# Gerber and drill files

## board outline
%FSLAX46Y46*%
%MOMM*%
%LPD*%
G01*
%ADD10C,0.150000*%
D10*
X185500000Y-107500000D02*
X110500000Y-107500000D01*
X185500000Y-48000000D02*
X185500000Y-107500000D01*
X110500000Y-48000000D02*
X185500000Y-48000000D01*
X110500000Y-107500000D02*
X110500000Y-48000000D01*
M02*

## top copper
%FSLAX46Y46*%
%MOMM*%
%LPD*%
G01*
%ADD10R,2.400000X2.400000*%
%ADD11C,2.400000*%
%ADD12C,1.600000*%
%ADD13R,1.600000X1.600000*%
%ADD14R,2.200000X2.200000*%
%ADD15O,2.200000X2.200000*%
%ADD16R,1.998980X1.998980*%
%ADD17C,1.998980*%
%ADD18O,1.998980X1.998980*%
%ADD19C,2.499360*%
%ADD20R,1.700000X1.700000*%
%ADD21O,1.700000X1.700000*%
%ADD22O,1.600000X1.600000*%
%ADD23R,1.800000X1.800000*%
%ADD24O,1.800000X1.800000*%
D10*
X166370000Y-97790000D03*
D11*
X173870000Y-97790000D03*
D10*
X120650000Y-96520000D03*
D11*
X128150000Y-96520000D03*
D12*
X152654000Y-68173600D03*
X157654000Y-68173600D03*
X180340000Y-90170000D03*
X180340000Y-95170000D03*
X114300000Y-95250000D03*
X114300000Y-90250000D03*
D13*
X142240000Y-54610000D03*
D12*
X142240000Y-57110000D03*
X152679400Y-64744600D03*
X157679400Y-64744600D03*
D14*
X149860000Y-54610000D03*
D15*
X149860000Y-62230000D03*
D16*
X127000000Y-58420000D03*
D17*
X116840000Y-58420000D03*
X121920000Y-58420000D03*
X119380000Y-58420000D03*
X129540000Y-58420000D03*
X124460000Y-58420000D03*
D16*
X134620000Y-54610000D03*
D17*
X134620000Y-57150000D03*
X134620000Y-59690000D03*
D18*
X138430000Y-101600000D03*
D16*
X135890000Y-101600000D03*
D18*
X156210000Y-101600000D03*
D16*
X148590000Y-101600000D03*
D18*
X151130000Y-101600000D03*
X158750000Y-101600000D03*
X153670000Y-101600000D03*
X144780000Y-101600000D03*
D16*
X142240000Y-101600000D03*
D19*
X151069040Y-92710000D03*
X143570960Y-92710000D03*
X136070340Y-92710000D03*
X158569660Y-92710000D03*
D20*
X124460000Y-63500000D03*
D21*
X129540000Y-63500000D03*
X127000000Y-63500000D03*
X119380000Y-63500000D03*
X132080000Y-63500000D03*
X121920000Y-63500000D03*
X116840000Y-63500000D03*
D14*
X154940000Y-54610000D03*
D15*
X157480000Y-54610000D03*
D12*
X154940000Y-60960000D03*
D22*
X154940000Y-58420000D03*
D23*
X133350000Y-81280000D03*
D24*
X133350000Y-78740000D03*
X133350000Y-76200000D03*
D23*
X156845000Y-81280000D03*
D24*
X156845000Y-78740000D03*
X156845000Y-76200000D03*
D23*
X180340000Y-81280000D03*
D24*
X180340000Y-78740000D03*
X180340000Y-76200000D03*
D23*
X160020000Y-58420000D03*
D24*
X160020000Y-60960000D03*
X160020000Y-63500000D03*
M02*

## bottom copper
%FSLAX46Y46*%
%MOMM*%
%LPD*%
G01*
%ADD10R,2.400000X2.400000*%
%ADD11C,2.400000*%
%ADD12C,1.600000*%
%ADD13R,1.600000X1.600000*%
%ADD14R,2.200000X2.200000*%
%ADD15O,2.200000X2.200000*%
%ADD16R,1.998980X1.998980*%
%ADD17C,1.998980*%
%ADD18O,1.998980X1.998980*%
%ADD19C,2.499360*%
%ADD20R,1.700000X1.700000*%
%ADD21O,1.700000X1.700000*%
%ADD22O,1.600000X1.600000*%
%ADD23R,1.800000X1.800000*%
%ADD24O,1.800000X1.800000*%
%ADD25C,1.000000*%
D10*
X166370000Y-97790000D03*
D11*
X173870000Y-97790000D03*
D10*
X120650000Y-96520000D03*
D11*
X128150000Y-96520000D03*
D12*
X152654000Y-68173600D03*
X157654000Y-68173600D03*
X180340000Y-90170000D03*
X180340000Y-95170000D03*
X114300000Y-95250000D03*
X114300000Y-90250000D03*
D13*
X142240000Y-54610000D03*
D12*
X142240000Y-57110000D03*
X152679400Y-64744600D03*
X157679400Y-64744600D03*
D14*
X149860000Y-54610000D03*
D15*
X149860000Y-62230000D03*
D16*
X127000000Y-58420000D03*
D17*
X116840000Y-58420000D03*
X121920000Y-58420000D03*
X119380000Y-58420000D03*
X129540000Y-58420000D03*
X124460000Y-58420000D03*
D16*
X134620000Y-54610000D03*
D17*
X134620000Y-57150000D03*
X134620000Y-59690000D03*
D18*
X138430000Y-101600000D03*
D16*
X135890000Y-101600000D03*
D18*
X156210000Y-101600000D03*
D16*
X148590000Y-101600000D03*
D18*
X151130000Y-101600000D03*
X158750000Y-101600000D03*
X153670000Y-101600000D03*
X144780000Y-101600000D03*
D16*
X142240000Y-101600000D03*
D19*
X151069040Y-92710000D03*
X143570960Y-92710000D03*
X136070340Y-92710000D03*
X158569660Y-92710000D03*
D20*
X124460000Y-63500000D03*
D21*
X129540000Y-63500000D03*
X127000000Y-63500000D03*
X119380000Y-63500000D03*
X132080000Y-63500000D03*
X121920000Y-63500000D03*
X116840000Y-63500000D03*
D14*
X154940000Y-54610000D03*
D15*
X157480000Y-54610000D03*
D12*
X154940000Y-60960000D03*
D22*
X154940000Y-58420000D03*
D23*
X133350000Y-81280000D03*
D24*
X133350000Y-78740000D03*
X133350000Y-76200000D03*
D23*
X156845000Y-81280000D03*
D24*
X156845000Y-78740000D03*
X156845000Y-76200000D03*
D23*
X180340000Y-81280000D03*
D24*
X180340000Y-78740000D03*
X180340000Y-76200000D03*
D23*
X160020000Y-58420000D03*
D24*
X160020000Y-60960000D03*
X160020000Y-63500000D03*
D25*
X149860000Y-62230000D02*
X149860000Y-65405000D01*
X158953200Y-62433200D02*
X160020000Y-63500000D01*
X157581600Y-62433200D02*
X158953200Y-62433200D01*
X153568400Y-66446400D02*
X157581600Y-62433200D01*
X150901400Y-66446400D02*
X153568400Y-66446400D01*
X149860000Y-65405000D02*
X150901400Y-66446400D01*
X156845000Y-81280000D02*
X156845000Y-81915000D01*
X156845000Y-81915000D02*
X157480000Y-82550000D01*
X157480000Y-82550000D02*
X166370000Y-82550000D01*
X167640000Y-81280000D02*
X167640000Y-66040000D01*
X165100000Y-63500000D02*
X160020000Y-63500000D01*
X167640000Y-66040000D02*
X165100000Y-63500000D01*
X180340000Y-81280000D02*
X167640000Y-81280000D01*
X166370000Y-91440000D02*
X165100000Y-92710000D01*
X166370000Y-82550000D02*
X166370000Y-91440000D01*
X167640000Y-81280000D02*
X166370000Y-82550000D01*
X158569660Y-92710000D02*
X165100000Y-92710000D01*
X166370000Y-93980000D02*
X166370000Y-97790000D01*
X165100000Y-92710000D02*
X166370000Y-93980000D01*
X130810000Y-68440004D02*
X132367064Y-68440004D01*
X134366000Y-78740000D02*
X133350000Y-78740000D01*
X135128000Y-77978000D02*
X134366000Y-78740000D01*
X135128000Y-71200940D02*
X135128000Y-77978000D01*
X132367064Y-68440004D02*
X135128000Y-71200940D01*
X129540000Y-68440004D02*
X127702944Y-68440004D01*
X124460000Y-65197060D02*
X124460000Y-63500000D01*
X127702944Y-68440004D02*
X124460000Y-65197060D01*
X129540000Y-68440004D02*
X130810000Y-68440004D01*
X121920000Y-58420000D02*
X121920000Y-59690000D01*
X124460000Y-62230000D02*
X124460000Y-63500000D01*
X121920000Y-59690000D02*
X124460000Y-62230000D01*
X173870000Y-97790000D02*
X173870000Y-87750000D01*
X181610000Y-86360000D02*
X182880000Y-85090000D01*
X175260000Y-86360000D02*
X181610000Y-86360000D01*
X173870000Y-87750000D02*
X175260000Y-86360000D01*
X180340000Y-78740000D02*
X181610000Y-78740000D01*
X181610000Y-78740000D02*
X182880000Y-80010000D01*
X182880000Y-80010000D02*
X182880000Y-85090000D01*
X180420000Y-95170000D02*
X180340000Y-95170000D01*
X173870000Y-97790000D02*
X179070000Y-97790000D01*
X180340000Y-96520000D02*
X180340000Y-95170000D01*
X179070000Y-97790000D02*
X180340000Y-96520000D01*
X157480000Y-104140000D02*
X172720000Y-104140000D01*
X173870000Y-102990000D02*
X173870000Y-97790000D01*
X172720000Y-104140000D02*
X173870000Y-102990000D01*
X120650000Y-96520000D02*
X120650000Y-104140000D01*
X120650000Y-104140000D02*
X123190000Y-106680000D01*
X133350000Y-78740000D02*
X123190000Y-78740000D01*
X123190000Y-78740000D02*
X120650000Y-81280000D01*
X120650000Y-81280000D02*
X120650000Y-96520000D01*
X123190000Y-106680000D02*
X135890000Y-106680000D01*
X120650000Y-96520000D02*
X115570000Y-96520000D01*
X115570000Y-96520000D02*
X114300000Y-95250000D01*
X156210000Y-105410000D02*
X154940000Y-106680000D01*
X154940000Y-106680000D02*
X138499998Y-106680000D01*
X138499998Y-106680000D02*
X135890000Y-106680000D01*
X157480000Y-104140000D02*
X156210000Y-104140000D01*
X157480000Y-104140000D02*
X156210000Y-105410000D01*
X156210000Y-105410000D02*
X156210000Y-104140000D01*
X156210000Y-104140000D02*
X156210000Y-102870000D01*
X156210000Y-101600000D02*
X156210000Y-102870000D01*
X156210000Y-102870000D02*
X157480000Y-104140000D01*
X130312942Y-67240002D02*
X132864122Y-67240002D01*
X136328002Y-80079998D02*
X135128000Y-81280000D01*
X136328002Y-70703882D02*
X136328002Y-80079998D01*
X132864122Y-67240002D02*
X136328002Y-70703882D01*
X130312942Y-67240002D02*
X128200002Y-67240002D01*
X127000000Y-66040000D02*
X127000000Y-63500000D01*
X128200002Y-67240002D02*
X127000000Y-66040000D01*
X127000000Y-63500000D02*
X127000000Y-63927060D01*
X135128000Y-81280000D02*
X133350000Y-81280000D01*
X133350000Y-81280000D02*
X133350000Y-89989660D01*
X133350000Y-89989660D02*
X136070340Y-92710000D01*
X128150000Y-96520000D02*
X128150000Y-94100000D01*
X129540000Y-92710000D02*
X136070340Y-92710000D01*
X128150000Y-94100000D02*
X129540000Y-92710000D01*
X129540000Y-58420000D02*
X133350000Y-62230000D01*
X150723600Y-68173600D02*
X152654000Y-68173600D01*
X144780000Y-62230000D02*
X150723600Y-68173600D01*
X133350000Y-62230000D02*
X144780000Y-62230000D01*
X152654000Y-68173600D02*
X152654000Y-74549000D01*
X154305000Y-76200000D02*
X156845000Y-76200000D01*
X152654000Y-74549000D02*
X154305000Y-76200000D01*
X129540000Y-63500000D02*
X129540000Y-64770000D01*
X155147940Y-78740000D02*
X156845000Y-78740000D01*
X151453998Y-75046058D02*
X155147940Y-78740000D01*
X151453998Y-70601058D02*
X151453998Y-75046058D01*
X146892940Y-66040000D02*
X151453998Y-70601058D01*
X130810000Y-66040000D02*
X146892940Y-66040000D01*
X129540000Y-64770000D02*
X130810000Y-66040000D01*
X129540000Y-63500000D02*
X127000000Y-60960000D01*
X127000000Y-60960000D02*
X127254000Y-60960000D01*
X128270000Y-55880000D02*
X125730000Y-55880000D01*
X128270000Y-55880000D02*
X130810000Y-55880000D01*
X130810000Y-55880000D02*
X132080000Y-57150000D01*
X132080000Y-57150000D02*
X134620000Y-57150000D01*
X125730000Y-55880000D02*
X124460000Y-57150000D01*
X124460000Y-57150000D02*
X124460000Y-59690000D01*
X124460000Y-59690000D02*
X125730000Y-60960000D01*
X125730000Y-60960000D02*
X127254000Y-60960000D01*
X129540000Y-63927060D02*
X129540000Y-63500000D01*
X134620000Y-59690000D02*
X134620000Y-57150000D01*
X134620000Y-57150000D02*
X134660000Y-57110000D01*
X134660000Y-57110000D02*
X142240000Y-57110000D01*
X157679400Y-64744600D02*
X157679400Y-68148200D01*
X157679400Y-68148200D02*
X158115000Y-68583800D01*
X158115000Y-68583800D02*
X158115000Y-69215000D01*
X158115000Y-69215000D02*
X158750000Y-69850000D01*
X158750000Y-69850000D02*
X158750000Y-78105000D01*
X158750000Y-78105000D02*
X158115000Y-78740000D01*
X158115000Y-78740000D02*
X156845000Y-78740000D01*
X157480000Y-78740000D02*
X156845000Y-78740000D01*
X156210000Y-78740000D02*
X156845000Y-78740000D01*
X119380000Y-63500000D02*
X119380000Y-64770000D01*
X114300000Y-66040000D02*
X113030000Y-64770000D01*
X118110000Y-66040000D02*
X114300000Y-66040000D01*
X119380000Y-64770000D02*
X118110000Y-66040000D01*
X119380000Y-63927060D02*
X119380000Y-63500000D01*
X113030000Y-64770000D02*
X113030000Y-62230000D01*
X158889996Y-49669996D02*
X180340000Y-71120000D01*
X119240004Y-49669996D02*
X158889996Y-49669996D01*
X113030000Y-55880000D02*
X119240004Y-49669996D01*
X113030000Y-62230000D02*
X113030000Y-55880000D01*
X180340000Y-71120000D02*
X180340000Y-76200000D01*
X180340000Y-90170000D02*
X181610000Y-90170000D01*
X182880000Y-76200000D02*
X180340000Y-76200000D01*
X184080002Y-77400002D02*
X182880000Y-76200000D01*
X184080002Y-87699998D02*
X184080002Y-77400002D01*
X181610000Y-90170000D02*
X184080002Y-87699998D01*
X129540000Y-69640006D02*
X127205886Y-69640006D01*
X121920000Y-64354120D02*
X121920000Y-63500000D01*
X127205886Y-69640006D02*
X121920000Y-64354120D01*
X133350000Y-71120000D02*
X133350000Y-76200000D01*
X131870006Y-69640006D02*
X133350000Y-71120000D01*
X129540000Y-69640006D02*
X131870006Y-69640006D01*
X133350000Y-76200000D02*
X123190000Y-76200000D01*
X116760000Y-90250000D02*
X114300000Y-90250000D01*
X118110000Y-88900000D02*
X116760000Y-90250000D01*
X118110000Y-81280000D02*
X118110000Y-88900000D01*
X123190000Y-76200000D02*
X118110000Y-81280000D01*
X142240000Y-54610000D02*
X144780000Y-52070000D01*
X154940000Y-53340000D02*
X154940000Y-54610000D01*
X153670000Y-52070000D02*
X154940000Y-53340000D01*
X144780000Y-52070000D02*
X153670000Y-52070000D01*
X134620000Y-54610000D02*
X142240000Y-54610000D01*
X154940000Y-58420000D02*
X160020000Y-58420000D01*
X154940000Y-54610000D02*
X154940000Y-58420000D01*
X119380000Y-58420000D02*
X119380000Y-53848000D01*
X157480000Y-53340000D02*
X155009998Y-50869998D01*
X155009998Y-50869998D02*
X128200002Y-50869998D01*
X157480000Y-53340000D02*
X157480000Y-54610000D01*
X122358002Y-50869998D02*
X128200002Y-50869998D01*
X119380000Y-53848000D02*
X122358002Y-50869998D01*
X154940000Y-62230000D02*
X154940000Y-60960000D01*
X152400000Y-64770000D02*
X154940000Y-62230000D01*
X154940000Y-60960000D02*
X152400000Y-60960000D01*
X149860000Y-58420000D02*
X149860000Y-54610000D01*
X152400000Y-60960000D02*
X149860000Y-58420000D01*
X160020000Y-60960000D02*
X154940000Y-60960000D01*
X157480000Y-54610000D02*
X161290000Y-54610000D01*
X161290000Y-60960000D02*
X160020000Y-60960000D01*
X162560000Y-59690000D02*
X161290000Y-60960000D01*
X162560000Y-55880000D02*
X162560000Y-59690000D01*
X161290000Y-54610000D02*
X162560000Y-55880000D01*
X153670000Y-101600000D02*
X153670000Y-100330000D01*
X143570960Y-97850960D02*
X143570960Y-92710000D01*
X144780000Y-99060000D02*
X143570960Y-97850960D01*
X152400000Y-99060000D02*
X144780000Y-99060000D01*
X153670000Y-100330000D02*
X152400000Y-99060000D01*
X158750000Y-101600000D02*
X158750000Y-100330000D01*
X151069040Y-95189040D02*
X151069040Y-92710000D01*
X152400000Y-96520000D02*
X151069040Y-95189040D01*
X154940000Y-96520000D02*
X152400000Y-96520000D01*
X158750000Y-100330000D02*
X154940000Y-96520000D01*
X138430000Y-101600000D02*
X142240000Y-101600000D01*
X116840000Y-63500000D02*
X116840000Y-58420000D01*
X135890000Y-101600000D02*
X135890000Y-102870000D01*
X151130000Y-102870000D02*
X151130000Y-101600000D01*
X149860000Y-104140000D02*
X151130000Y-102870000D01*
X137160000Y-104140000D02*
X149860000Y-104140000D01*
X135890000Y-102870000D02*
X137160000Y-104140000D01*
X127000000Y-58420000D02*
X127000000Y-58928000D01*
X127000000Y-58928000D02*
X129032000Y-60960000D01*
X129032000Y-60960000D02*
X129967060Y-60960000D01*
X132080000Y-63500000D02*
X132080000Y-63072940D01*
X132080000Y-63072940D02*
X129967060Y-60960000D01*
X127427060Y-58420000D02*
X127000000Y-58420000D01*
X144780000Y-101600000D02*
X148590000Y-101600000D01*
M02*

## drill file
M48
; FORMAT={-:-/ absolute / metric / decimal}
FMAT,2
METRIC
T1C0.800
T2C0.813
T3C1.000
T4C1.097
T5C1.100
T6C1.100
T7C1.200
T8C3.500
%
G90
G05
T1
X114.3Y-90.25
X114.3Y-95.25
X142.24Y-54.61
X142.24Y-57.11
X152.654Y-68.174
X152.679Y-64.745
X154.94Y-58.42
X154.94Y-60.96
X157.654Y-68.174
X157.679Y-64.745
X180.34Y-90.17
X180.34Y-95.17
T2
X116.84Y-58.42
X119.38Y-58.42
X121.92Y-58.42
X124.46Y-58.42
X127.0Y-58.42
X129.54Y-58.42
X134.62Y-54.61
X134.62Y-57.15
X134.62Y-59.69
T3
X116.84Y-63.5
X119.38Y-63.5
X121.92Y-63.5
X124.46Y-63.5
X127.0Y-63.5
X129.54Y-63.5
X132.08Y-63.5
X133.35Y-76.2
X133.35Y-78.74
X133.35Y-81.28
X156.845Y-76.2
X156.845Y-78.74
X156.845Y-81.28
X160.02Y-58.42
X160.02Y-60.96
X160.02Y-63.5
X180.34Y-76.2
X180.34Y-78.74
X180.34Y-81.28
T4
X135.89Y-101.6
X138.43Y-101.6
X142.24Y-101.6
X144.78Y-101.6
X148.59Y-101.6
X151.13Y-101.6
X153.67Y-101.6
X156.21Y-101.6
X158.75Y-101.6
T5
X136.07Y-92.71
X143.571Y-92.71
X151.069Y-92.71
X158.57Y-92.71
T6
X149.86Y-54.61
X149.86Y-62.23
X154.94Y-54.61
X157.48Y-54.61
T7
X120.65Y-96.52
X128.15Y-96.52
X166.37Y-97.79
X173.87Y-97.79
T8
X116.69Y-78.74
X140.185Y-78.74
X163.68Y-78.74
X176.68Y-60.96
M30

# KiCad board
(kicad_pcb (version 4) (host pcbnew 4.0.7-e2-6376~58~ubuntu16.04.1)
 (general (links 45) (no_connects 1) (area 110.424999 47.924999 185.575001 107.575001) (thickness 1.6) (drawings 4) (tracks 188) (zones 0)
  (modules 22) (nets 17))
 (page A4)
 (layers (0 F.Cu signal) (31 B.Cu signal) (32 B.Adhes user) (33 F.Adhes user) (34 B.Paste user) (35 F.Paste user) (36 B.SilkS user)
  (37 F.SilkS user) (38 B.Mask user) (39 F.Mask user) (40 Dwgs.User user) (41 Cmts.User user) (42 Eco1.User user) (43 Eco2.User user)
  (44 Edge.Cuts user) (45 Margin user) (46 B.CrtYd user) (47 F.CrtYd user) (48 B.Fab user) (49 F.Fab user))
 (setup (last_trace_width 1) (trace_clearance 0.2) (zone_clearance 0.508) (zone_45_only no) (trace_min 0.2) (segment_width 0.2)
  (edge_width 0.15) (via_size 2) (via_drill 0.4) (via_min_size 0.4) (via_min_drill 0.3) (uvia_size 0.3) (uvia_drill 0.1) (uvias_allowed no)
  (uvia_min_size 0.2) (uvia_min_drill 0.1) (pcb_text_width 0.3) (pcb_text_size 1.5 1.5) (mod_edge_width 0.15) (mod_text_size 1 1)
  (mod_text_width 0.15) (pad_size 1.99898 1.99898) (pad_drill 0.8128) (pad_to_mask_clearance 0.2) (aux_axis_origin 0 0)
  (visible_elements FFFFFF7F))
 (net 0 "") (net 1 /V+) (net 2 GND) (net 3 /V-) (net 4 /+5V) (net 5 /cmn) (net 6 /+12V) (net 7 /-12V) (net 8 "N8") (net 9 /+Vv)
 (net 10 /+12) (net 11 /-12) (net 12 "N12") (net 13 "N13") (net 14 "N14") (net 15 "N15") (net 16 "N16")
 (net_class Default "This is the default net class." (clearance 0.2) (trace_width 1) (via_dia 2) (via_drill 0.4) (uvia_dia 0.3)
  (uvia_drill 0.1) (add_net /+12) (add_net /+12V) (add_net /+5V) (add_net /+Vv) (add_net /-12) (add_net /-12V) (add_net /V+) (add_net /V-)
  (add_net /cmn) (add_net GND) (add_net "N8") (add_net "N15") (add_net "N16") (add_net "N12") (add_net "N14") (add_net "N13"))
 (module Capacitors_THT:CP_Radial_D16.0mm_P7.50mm (layer F.Cu) (at 166.37 97.79)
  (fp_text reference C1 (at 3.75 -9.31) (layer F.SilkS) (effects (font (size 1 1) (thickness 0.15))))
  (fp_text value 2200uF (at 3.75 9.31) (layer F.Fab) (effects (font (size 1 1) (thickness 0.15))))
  (pad 1 thru_hole rect (at 0 0) (size 2.4 2.4) (drill 1.2) (layers *.Cu *.Mask) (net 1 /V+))
  (pad 2 thru_hole circle (at 7.5 0) (size 2.4 2.4) (drill 1.2) (layers *.Cu *.Mask) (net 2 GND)))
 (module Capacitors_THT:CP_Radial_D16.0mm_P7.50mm (layer F.Cu) (at 120.65 96.52)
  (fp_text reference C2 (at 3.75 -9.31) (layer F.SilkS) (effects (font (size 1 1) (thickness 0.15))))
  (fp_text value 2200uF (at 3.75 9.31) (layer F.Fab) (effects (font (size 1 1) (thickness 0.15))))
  (pad 1 thru_hole rect (at 0 0) (size 2.4 2.4) (drill 1.2) (layers *.Cu *.Mask) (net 2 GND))
  (pad 2 thru_hole circle (at 7.5 0) (size 2.4 2.4) (drill 1.2) (layers *.Cu *.Mask) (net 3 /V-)))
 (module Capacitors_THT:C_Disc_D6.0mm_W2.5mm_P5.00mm (layer F.Cu) (at 152.654 68.1736)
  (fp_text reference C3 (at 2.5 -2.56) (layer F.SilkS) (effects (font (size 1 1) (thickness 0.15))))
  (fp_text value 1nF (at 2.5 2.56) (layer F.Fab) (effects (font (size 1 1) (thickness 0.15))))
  (pad 1 thru_hole circle (at 0 0) (size 1.6 1.6) (drill 0.8) (layers *.Cu *.Mask) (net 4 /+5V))
  (pad 2 thru_hole circle (at 5 0) (size 1.6 1.6) (drill 0.8) (layers *.Cu *.Mask) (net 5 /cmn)))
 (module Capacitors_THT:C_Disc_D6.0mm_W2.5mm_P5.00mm (layer F.Cu) (at 180.34 90.17 270)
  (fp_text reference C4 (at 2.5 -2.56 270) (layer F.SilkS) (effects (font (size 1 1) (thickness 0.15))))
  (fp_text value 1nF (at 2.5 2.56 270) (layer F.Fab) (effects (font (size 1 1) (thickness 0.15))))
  (pad 1 thru_hole circle (at 0 0 270) (size 1.6 1.6) (drill 0.8) (layers *.Cu *.Mask) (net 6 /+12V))
  (pad 2 thru_hole circle (at 5 0 270) (size 1.6 1.6) (drill 0.8) (layers *.Cu *.Mask) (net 2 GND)))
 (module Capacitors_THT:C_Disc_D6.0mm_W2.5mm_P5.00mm (layer F.Cu) (at 114.3 95.25 90)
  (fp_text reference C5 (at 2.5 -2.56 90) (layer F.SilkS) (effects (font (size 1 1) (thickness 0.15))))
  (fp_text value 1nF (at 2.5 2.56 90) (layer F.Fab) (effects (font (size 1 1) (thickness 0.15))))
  (pad 1 thru_hole circle (at 0 0 90) (size 1.6 1.6) (drill 0.8) (layers *.Cu *.Mask) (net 2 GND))
  (pad 2 thru_hole circle (at 5 0 90) (size 1.6 1.6) (drill 0.8) (layers *.Cu *.Mask) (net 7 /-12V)))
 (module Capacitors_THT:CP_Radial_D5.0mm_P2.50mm (layer F.Cu) (at 142.24 54.61 270)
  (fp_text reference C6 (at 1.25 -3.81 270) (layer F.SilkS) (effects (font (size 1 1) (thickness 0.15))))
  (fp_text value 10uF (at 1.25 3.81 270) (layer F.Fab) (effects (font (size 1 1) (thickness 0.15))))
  (pad 1 thru_hole rect (at 0 0 270) (size 1.6 1.6) (drill 0.8) (layers *.Cu *.Mask) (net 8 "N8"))
  (pad 2 thru_hole circle (at 2.5 0 270) (size 1.6 1.6) (drill 0.8) (layers *.Cu *.Mask) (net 5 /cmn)))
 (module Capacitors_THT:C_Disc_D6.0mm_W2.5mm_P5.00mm (layer F.Cu) (at 152.6794 64.7446)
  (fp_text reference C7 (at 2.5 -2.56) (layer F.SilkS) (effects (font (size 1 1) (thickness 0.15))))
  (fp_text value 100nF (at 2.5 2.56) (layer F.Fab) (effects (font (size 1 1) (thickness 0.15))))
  (pad 1 thru_hole circle (at 0 0) (size 1.6 1.6) (drill 0.8) (layers *.Cu *.Mask) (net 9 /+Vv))
  (pad 2 thru_hole circle (at 5 0) (size 1.6 1.6) (drill 0.8) (layers *.Cu *.Mask) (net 5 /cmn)))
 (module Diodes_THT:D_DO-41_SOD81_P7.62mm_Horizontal (layer F.Cu) (at 149.86 54.61 270)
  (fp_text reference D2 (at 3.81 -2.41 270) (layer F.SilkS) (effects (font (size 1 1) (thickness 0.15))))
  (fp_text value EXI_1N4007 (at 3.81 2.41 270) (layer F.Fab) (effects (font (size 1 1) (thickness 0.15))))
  (pad 1 thru_hole rect (at 0 0 270) (size 2.2 2.2) (drill 1.1) (layers *.Cu *.Mask) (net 9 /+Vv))
  (pad 2 thru_hole oval (at 7.62 0 270) (size 2.2 2.2) (drill 1.1) (layers *.Cu *.Mask) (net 1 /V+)))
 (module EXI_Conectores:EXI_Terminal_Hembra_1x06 (layer F.Cu) (at 123.19 58.42 180)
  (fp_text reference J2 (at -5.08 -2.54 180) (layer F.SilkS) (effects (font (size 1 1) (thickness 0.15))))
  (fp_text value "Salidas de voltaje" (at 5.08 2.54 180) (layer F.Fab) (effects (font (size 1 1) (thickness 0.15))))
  (pad 1 thru_hole rect (at -3.81 0 180) (size 1.99898 1.99898) (drill 0.8128) (layers *.Cu *.Mask F.SilkS) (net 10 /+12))
  (pad 2 thru_hole circle (at 6.35 0 180) (size 1.99898 1.99898) (drill 0.8128) (layers *.Cu *.Mask F.SilkS) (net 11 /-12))
  (pad 3 thru_hole circle (at 1.27 0 180) (size 1.99898 1.99898) (drill 0.8128) (layers *.Cu *.Mask F.SilkS) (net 2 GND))
  (pad 4 thru_hole circle (at 3.81 0 180) (size 1.99898 1.99898) (drill 0.8128) (layers *.Cu *.Mask F.SilkS) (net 9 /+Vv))
  (pad 5 thru_hole circle (at -6.35 0 180) (size 1.99898 1.99898) (drill 0.8128) (layers *.Cu *.Mask F.SilkS) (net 4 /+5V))
  (pad 6 thru_hole circle (at -1.27 0 180) (size 1.99898 1.99898) (drill 0.8128) (layers *.Cu *.Mask F.SilkS) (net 5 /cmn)))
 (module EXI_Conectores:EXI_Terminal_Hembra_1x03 (layer F.Cu) (at 134.62 57.15 270)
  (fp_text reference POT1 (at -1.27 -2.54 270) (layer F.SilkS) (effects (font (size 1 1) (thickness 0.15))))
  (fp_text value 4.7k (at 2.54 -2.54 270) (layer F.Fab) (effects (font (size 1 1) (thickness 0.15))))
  (pad 1 thru_hole rect (at -2.54 0 270) (size 1.99898 1.99898) (drill 0.8128) (layers *.Cu *.Mask F.SilkS) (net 8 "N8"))
  (pad 2 thru_hole circle (at 0 0 270) (size 1.99898 1.99898) (drill 0.8128) (layers *.Cu *.Mask F.SilkS) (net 5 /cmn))
  (pad 3 thru_hole circle (at 2.54 0 270) (size 1.99898 1.99898) (drill 0.8128) (layers *.Cu *.Mask F.SilkS) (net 5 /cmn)))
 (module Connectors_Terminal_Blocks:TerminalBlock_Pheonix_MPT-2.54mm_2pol (layer F.Cu) (at 135.89 101.6)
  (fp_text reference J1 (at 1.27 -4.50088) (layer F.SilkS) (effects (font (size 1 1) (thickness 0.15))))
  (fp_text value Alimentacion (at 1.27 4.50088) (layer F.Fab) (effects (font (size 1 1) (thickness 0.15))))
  (pad 2 thru_hole oval (at 2.54 0) (size 1.99898 1.99898) (drill 1.09728) (layers *.Cu *.Mask) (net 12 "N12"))
  (pad 1 thru_hole rect (at 0 0) (size 1.99898 1.99898) (drill 1.09728) (layers *.Cu *.Mask) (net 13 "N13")))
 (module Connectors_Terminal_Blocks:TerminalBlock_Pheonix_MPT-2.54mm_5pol (layer F.Cu) (at 148.59 101.6)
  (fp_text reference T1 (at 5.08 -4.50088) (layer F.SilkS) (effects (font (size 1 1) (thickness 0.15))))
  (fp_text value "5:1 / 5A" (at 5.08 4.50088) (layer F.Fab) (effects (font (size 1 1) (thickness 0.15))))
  (pad 4 thru_hole oval (at 7.62 0 180) (size 1.99898 1.99898) (drill 1.09728) (layers *.Cu *.Mask) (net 2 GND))
  (pad 1 thru_hole rect (at 0 0 180) (size 1.99898 1.99898) (drill 1.09728) (layers *.Cu *.Mask) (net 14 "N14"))
  (pad 2 thru_hole oval (at 2.54 0 180) (size 1.99898 1.99898) (drill 1.09728) (layers *.Cu *.Mask) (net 13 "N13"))
  (pad 3 thru_hole oval (at 10.16 0 180) (size 1.99898 1.99898) (drill 1.09728) (layers *.Cu *.Mask) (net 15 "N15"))
  (pad 5 thru_hole oval (at 5.08 0 180) (size 1.99898 1.99898) (drill 1.09728) (layers *.Cu *.Mask) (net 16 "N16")))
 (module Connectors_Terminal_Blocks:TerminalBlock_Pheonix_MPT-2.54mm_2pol (layer F.Cu) (at 142.24 101.6)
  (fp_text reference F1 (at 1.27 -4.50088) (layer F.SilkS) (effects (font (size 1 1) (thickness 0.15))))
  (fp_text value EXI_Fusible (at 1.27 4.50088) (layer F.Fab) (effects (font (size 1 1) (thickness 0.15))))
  (pad 2 thru_hole oval (at 2.54 0) (size 1.99898 1.99898) (drill 1.09728) (layers *.Cu *.Mask) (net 14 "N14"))
  (pad 1 thru_hole rect (at 0 0) (size 1.99898 1.99898) (drill 1.09728) (layers *.Cu *.Mask) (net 12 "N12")))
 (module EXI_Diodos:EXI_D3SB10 (layer F.Cu) (at 147.32 92.71 180)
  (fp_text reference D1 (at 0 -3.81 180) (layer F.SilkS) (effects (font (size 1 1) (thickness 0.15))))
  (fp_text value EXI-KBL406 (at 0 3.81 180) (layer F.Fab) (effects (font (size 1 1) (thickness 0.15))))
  (pad 2 thru_hole circle (at -3.74904 0 180) (size 2.49936 2.49936) (drill 1.09982) (layers *.Cu *.Mask F.SilkS) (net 15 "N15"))
  (pad 3 thru_hole circle (at 3.74904 0 180) (size 2.49936 2.49936) (drill 1.09982) (layers *.Cu *.Mask F.SilkS) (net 16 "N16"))
  (pad 4 thru_hole circle (at 11.24966 0 180) (size 2.49936 2.49936) (drill 1.09982) (layers *.Cu *.Mask F.SilkS) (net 3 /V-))
  (pad 1 thru_hole circle (at -11.24966 0 180) (size 2.49936 2.49936) (drill 1.09982) (layers *.Cu *.Mask F.SilkS) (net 1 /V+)))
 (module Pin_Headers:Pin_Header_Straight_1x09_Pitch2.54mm (layer F.Cu) (at 137.16 63.5 270)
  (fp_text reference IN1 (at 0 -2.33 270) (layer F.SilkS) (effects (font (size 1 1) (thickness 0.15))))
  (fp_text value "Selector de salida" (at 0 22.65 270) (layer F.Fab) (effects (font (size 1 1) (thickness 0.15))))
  (pad 1 thru_hole rect (at 0 12.7 270) (size 1.7 1.7) (drill 1) (layers *.Cu *.Mask) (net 2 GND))
  (pad 2 thru_hole oval (at 0 7.62 270) (size 1.7 1.7) (drill 1) (layers *.Cu *.Mask) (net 5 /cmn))
  (pad 3 thru_hole oval (at 0 10.16 270) (size 1.7 1.7) (drill 1) (layers *.Cu *.Mask) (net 3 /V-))
  (pad 4 thru_hole oval (at 0 17.78 270) (size 1.7 1.7) (drill 1) (layers *.Cu *.Mask) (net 6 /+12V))
  (pad 5 thru_hole oval (at 0 5.08 270) (size 1.7 1.7) (drill 1) (layers *.Cu *.Mask) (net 10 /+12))
  (pad 7 thru_hole oval (at 0 15.24 270) (size 1.7 1.7) (drill 1) (layers *.Cu *.Mask) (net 7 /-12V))
  (pad 8 thru_hole oval (at 0 20.32 270) (size 1.7 1.7) (drill 1) (layers *.Cu *.Mask) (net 11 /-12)))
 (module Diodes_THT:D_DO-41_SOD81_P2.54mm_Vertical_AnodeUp (layer F.Cu) (at 154.94 54.61)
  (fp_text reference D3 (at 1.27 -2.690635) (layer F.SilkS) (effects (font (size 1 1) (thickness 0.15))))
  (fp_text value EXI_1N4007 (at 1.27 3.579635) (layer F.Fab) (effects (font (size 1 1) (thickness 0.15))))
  (pad 1 thru_hole rect (at 0 0) (size 2.2 2.2) (drill 1.1) (layers *.Cu *.Mask) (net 8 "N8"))
  (pad 2 thru_hole oval (at 2.54 0) (size 2.2 2.2) (drill 1.1) (layers *.Cu *.Mask) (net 9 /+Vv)))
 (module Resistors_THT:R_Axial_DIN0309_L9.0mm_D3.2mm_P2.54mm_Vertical (layer F.Cu) (at 154.94 60.96 90)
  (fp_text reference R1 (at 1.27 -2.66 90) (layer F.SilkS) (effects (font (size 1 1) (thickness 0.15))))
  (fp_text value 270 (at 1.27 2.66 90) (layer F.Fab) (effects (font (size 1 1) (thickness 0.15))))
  (pad 1 thru_hole circle (at 0 0 90) (size 1.6 1.6) (drill 0.8) (layers *.Cu *.Mask) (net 9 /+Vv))
  (pad 2 thru_hole oval (at 2.54 0 90) (size 1.6 1.6) (drill 0.8) (layers *.Cu *.Mask) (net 8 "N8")))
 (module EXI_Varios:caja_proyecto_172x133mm (layer F.Cu) (at 149 110.5 90)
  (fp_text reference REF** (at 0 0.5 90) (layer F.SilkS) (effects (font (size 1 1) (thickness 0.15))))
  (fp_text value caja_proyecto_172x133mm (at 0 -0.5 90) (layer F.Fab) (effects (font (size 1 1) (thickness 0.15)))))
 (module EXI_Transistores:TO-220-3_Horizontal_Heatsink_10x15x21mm (layer F.Cu) (at 133.35 78.74 90)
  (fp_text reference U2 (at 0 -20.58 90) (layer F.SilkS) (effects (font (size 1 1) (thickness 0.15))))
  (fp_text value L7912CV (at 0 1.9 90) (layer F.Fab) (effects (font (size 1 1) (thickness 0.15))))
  (pad 0 np_thru_hole oval (at 0 -16.66 90) (size 3.5 3.5) (drill 3.5) (layers *.Cu *.Mask))
  (pad 1 thru_hole rect (at -2.54 0 90) (size 1.8 1.8) (drill 1) (layers *.Cu *.Mask) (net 3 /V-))
  (pad 2 thru_hole oval (at 0 0 90) (size 1.8 1.8) (drill 1) (layers *.Cu *.Mask) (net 2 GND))
  (pad 3 thru_hole oval (at 2.54 0 90) (size 1.8 1.8) (drill 1) (layers *.Cu *.Mask) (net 7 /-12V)))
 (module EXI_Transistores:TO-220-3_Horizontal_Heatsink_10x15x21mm (layer F.Cu) (at 156.845 78.74 90)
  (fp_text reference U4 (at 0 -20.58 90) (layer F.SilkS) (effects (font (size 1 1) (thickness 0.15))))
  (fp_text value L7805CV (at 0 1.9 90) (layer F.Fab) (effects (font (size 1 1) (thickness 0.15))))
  (pad 0 np_thru_hole oval (at 0 -16.66 90) (size 3.5 3.5) (drill 3.5) (layers *.Cu *.Mask))
  (pad 1 thru_hole rect (at -2.54 0 90) (size 1.8 1.8) (drill 1) (layers *.Cu *.Mask) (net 1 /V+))
  (pad 2 thru_hole oval (at 0 0 90) (size 1.8 1.8) (drill 1) (layers *.Cu *.Mask) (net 5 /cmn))
  (pad 3 thru_hole oval (at 2.54 0 90) (size 1.8 1.8) (drill 1) (layers *.Cu *.Mask) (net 4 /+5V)))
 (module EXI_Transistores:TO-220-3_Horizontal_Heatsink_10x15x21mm (layer F.Cu) (at 180.34 78.74 90)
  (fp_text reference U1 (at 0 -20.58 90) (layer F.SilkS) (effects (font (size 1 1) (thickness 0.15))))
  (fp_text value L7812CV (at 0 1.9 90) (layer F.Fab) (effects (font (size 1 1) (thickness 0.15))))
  (pad 0 np_thru_hole oval (at 0 -16.66 90) (size 3.5 3.5) (drill 3.5) (layers *.Cu *.Mask))
  (pad 1 thru_hole rect (at -2.54 0 90) (size 1.8 1.8) (drill 1) (layers *.Cu *.Mask) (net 1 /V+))
  (pad 2 thru_hole oval (at 0 0 90) (size 1.8 1.8) (drill 1) (layers *.Cu *.Mask) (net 2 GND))
  (pad 3 thru_hole oval (at 2.54 0 90) (size 1.8 1.8) (drill 1) (layers *.Cu *.Mask) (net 6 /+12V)))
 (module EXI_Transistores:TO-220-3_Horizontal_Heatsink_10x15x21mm (layer F.Cu) (at 160.02 60.96 270)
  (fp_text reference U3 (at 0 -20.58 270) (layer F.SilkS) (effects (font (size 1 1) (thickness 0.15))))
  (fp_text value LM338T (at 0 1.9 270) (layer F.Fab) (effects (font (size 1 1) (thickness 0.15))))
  (pad 0 np_thru_hole oval (at 0 -16.66 270) (size 3.5 3.5) (drill 3.5) (layers *.Cu *.Mask))
  (pad 1 thru_hole rect (at -2.54 0 270) (size 1.8 1.8) (drill 1) (layers *.Cu *.Mask) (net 8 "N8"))
  (pad 2 thru_hole oval (at 0 0 270) (size 1.8 1.8) (drill 1) (layers *.Cu *.Mask) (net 9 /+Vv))
  (pad 3 thru_hole oval (at 2.54 0 270) (size 1.8 1.8) (drill 1) (layers *.Cu *.Mask) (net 1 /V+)))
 (gr_line (start 185.5 107.5) (end 110.5 107.5) (angle 90) (layer Edge.Cuts) (width 0.15))
 (gr_line (start 185.5 48) (end 185.5 107.5) (angle 90) (layer Edge.Cuts) (width 0.15))
 (gr_line (start 110.5 48) (end 185.5 48) (angle 90) (layer Edge.Cuts) (width 0.15))
 (gr_line (start 110.5 107.5) (end 110.5 48) (angle 90) (layer Edge.Cuts) (width 0.15))
 (segment (start 149.86 62.23) (end 149.86 65.405) (width 1) (layer B.Cu) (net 1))
 (segment (start 158.9532 62.4332) (end 160.02 63.5) (width 1) (layer B.Cu) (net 1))
 (segment (start 157.5816 62.4332) (end 158.9532 62.4332) (width 1) (layer B.Cu) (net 1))
 (segment (start 153.5684 66.4464) (end 157.5816 62.4332) (width 1) (layer B.Cu) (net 1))
 (segment (start 150.9014 66.4464) (end 153.5684 66.4464) (width 1) (layer B.Cu) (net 1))
 (segment (start 149.86 65.405) (end 150.9014 66.4464) (width 1) (layer B.Cu) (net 1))
 (segment (start 156.845 81.28) (end 156.845 81.915) (width 1) (layer B.Cu) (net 1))
 (segment (start 156.845 81.915) (end 157.48 82.55) (width 1) (layer B.Cu) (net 1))
 (segment (start 157.48 82.55) (end 166.37 82.55) (width 1) (layer B.Cu) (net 1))
 (segment (start 167.64 81.28) (end 167.64 66.04) (width 1) (layer B.Cu) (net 1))
 (segment (start 165.1 63.5) (end 160.02 63.5) (width 1) (layer B.Cu) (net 1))
 (segment (start 167.64 66.04) (end 165.1 63.5) (width 1) (layer B.Cu) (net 1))
 (segment (start 180.34 81.28) (end 167.64 81.28) (width 1) (layer B.Cu) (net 1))
 (segment (start 166.37 91.44) (end 165.1 92.71) (width 1) (layer B.Cu) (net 1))
 (segment (start 166.37 82.55) (end 166.37 91.44) (width 1) (layer B.Cu) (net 1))
 (segment (start 167.64 81.28) (end 166.37 82.55) (width 1) (layer B.Cu) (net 1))
 (segment (start 158.56966 92.71) (end 165.1 92.71) (width 1) (layer B.Cu) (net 1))
 (segment (start 166.37 93.98) (end 166.37 97.79) (width 1) (layer B.Cu) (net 1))
 (segment (start 165.1 92.71) (end 166.37 93.98) (width 1) (layer B.Cu) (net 1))
 (segment (start 130.81 68.440004) (end 132.367064 68.440004) (width 1) (layer B.Cu) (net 2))
 (segment (start 134.366 78.74) (end 133.35 78.74) (width 1) (layer B.Cu) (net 2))
 (segment (start 135.128 77.978) (end 134.366 78.74) (width 1) (layer B.Cu) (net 2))
 (segment (start 135.128 71.20094) (end 135.128 77.978) (width 1) (layer B.Cu) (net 2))
 (segment (start 132.367064 68.440004) (end 135.128 71.20094) (width 1) (layer B.Cu) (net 2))
 (segment (start 129.54 68.440004) (end 127.702944 68.440004) (width 1) (layer B.Cu) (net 2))
 (segment (start 124.46 65.19706) (end 124.46 63.5) (width 1) (layer B.Cu) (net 2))
 (segment (start 127.702944 68.440004) (end 124.46 65.19706) (width 1) (layer B.Cu) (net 2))
 (segment (start 129.54 68.440004) (end 130.81 68.440004) (width 1) (layer B.Cu) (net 2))
 (segment (start 121.92 58.42) (end 121.92 59.69) (width 1) (layer B.Cu) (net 2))
 (segment (start 124.46 62.23) (end 124.46 63.5) (width 1) (layer B.Cu) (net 2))
 (segment (start 121.92 59.69) (end 124.46 62.23) (width 1) (layer B.Cu) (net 2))
 (segment (start 173.87 97.79) (end 173.87 87.75) (width 1) (layer B.Cu) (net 2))
 (segment (start 181.61 86.36) (end 182.88 85.09) (width 1) (layer B.Cu) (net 2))
 (segment (start 175.26 86.36) (end 181.61 86.36) (width 1) (layer B.Cu) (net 2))
 (segment (start 173.87 87.75) (end 175.26 86.36) (width 1) (layer B.Cu) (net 2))
 (segment (start 180.34 78.74) (end 181.61 78.74) (width 1) (layer B.Cu) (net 2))
 (segment (start 181.61 78.74) (end 182.88 80.01) (width 1) (layer B.Cu) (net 2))
 (segment (start 182.88 80.01) (end 182.88 85.09) (width 1) (layer B.Cu) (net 2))
 (segment (start 180.42 95.17) (end 180.34 95.17) (width 1) (layer B.Cu) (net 2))
 (segment (start 173.87 97.79) (end 179.07 97.79) (width 1) (layer B.Cu) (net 2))
 (segment (start 180.34 96.52) (end 180.34 95.17) (width 1) (layer B.Cu) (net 2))
 (segment (start 179.07 97.79) (end 180.34 96.52) (width 1) (layer B.Cu) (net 2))
 (segment (start 157.48 104.14) (end 172.72 104.14) (width 1) (layer B.Cu) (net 2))
 (segment (start 173.87 102.99) (end 173.87 97.79) (width 1) (layer B.Cu) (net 2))
 (segment (start 172.72 104.14) (end 173.87 102.99) (width 1) (layer B.Cu) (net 2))
 (segment (start 120.65 96.52) (end 120.65 104.14) (width 1) (layer B.Cu) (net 2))
 (segment (start 120.65 104.14) (end 123.19 106.68) (width 1) (layer B.Cu) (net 2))
 (segment (start 133.35 78.74) (end 123.19 78.74) (width 1) (layer B.Cu) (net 2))
 (segment (start 123.19 78.74) (end 120.65 81.28) (width 1) (layer B.Cu) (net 2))
 (segment (start 120.65 81.28) (end 120.65 96.52) (width 1) (layer B.Cu) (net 2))
 (segment (start 123.19 106.68) (end 135.89 106.68) (width 1) (layer B.Cu) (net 2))
 (segment (start 120.65 96.52) (end 115.57 96.52) (width 1) (layer B.Cu) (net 2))
 (segment (start 115.57 96.52) (end 114.3 95.25) (width 1) (layer B.Cu) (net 2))
 (segment (start 156.21 105.41) (end 154.94 106.68) (width 1) (layer B.Cu) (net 2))
 (segment (start 154.94 106.68) (end 138.499998 106.68) (width 1) (layer B.Cu) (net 2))
 (segment (start 138.499998 106.68) (end 135.89 106.68) (width 1) (layer B.Cu) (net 2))
 (segment (start 157.48 104.14) (end 156.21 104.14) (width 1) (layer B.Cu) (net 2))
 (segment (start 157.48 104.14) (end 156.21 105.41) (width 1) (layer B.Cu) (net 2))
 (segment (start 156.21 105.41) (end 156.21 104.14) (width 1) (layer B.Cu) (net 2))
 (segment (start 156.21 104.14) (end 156.21 102.87) (width 1) (layer B.Cu) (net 2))
 (segment (start 156.21 101.6) (end 156.21 102.87) (width 1) (layer B.Cu) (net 2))
 (segment (start 156.21 102.87) (end 157.48 104.14) (width 1) (layer B.Cu) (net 2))
 (segment (start 130.312942 67.240002) (end 132.864122 67.240002) (width 1) (layer B.Cu) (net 3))
 (segment (start 136.328002 80.079998) (end 135.128 81.28) (width 1) (layer B.Cu) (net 3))
 (segment (start 136.328002 70.703882) (end 136.328002 80.079998) (width 1) (layer B.Cu) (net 3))
 (segment (start 132.864122 67.240002) (end 136.328002 70.703882) (width 1) (layer B.Cu) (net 3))
 (segment (start 130.312942 67.240002) (end 128.200002 67.240002) (width 1) (layer B.Cu) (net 3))
 (segment (start 127 66.04) (end 127 63.5) (width 1) (layer B.Cu) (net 3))
 (segment (start 128.200002 67.240002) (end 127 66.04) (width 1) (layer B.Cu) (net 3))
 (segment (start 127 63.5) (end 127 63.92706) (width 1) (layer B.Cu) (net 3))
 (segment (start 135.128 81.28) (end 133.35 81.28) (width 1) (layer B.Cu) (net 3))
 (segment (start 133.35 81.28) (end 133.35 89.98966) (width 1) (layer B.Cu) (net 3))
 (segment (start 133.35 89.98966) (end 136.07034 92.71) (width 1) (layer B.Cu) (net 3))
 (segment (start 128.15 96.52) (end 128.15 94.1) (width 1) (layer B.Cu) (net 3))
 (segment (start 129.54 92.71) (end 136.07034 92.71) (width 1) (layer B.Cu) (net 3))
 (segment (start 128.15 94.1) (end 129.54 92.71) (width 1) (layer B.Cu) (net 3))
 (segment (start 129.54 58.42) (end 133.35 62.23) (width 1) (layer B.Cu) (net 4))
 (segment (start 150.7236 68.1736) (end 152.654 68.1736) (width 1) (layer B.Cu) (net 4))
 (segment (start 144.78 62.23) (end 150.7236 68.1736) (width 1) (layer B.Cu) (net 4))
 (segment (start 133.35 62.23) (end 144.78 62.23) (width 1) (layer B.Cu) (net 4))
 (segment (start 152.654 68.1736) (end 152.654 74.549) (width 1) (layer B.Cu) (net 4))
 (segment (start 154.305 76.2) (end 156.845 76.2) (width 1) (layer B.Cu) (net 4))
 (segment (start 152.654 74.549) (end 154.305 76.2) (width 1) (layer B.Cu) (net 4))
 (segment (start 129.54 63.5) (end 129.54 64.77) (width 1) (layer B.Cu) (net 5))
 (segment (start 155.14794 78.74) (end 156.845 78.74) (width 1) (layer B.Cu) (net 5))
 (segment (start 151.453998 75.046058) (end 155.14794 78.74) (width 1) (layer B.Cu) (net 5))
 (segment (start 151.453998 70.601058) (end 151.453998 75.046058) (width 1) (layer B.Cu) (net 5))
 (segment (start 146.89294 66.04) (end 151.453998 70.601058) (width 1) (layer B.Cu) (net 5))
 (segment (start 130.81 66.04) (end 146.89294 66.04) (width 1) (layer B.Cu) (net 5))
 (segment (start 129.54 64.77) (end 130.81 66.04) (width 1) (layer B.Cu) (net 5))
 (segment (start 129.54 63.5) (end 127 60.96) (width 1) (layer B.Cu) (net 5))
 (segment (start 127 60.96) (end 127.254 60.96) (width 1) (layer B.Cu) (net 5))
 (segment (start 128.27 55.88) (end 125.73 55.88) (width 1) (layer B.Cu) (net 5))
 (segment (start 128.27 55.88) (end 130.81 55.88) (width 1) (layer B.Cu) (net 5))
 (segment (start 130.81 55.88) (end 132.08 57.15) (width 1) (layer B.Cu) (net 5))
 (segment (start 132.08 57.15) (end 134.62 57.15) (width 1) (layer B.Cu) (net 5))
 (segment (start 125.73 55.88) (end 124.46 57.15) (width 1) (layer B.Cu) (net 5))
 (segment (start 124.46 57.15) (end 124.46 59.69) (width 1) (layer B.Cu) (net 5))
 (segment (start 124.46 59.69) (end 125.73 60.96) (width 1) (layer B.Cu) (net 5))
 (segment (start 125.73 60.96) (end 127.254 60.96) (width 1) (layer B.Cu) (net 5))
 (segment (start 129.54 63.92706) (end 129.54 63.5) (width 1) (layer B.Cu) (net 5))
 (segment (start 134.62 59.69) (end 134.62 57.15) (width 1) (layer B.Cu) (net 5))
 (segment (start 134.62 57.15) (end 134.66 57.11) (width 1) (layer B.Cu) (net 5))
 (segment (start 134.66 57.11) (end 142.24 57.11) (width 1) (layer B.Cu) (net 5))
 (segment (start 157.6794 64.7446) (end 157.6794 68.1482) (width 1) (layer B.Cu) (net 5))
 (segment (start 157.6794 68.1482) (end 158.115 68.5838) (width 1) (layer B.Cu) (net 5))
 (segment (start 158.115 68.5838) (end 158.115 69.215) (width 1) (layer B.Cu) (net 5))
 (segment (start 158.115 69.215) (end 158.75 69.85) (width 1) (layer B.Cu) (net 5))
 (segment (start 158.75 69.85) (end 158.75 78.105) (width 1) (layer B.Cu) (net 5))
 (segment (start 158.75 78.105) (end 158.115 78.74) (width 1) (layer B.Cu) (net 5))
 (segment (start 158.115 78.74) (end 156.845 78.74) (width 1) (layer B.Cu) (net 5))
 (segment (start 157.48 78.74) (end 156.845 78.74) (width 1) (layer B.Cu) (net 5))
 (segment (start 156.21 78.74) (end 156.845 78.74) (width 1) (layer B.Cu) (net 5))
 (segment (start 119.38 63.5) (end 119.38 64.77) (width 1) (layer B.Cu) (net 6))
 (segment (start 114.3 66.04) (end 113.03 64.77) (width 1) (layer B.Cu) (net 6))
 (segment (start 118.11 66.04) (end 114.3 66.04) (width 1) (layer B.Cu) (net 6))
 (segment (start 119.38 64.77) (end 118.11 66.04) (width 1) (layer B.Cu) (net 6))
 (segment (start 119.38 63.92706) (end 119.38 63.5) (width 1) (layer B.Cu) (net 6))
 (segment (start 113.03 64.77) (end 113.03 62.23) (width 1) (layer B.Cu) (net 6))
 (segment (start 158.889996 49.669996) (end 180.34 71.12) (width 1) (layer B.Cu) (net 6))
 (segment (start 119.240004 49.669996) (end 158.889996 49.669996) (width 1) (layer B.Cu) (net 6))
 (segment (start 113.03 55.88) (end 119.240004 49.669996) (width 1) (layer B.Cu) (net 6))
 (segment (start 113.03 62.23) (end 113.03 55.88) (width 1) (layer B.Cu) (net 6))
 (segment (start 180.34 71.12) (end 180.34 76.2) (width 1) (layer B.Cu) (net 6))
 (segment (start 180.34 90.17) (end 181.61 90.17) (width 1) (layer B.Cu) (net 6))
 (segment (start 182.88 76.2) (end 180.34 76.2) (width 1) (layer B.Cu) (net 6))
 (segment (start 184.080002 77.400002) (end 182.88 76.2) (width 1) (layer B.Cu) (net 6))
 (segment (start 184.080002 87.699998) (end 184.080002 77.400002) (width 1) (layer B.Cu) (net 6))
 (segment (start 181.61 90.17) (end 184.080002 87.699998) (width 1) (layer B.Cu) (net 6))
 (segment (start 129.54 69.640006) (end 127.205886 69.640006) (width 1) (layer B.Cu) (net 7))
 (segment (start 121.92 64.35412) (end 121.92 63.5) (width 1) (layer B.Cu) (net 7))
 (segment (start 127.205886 69.640006) (end 121.92 64.35412) (width 1) (layer B.Cu) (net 7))
 (segment (start 133.35 71.12) (end 133.35 76.2) (width 1) (layer B.Cu) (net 7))
 (segment (start 131.870006 69.640006) (end 133.35 71.12) (width 1) (layer B.Cu) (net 7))
 (segment (start 129.54 69.640006) (end 131.870006 69.640006) (width 1) (layer B.Cu) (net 7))
 (segment (start 133.35 76.2) (end 123.19 76.2) (width 1) (layer B.Cu) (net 7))
 (segment (start 116.76 90.25) (end 114.3 90.25) (width 1) (layer B.Cu) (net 7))
 (segment (start 118.11 88.9) (end 116.76 90.25) (width 1) (layer B.Cu) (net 7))
 (segment (start 118.11 81.28) (end 118.11 88.9) (width 1) (layer B.Cu) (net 7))
 (segment (start 123.19 76.2) (end 118.11 81.28) (width 1) (layer B.Cu) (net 7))
 (segment (start 142.24 54.61) (end 144.78 52.07) (width 1) (layer B.Cu) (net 8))
 (segment (start 154.94 53.34) (end 154.94 54.61) (width 1) (layer B.Cu) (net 8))
 (segment (start 153.67 52.07) (end 154.94 53.34) (width 1) (layer B.Cu) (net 8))
 (segment (start 144.78 52.07) (end 153.67 52.07) (width 1) (layer B.Cu) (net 8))
 (segment (start 134.62 54.61) (end 142.24 54.61) (width 1) (layer B.Cu) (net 8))
 (segment (start 154.94 58.42) (end 160.02 58.42) (width 1) (layer B.Cu) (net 8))
 (segment (start 154.94 54.61) (end 154.94 58.42) (width 1) (layer B.Cu) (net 8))
 (segment (start 119.38 58.42) (end 119.38 53.848) (width 1) (layer B.Cu) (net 9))
 (segment (start 157.48 53.34) (end 155.009998 50.869998) (width 1) (layer B.Cu) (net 9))
 (segment (start 155.009998 50.869998) (end 128.200002 50.869998) (width 1) (layer B.Cu) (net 9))
 (segment (start 157.48 53.34) (end 157.48 54.61) (width 1) (layer B.Cu) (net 9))
 (segment (start 122.358002 50.869998) (end 128.200002 50.869998) (width 1) (layer B.Cu) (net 9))
 (segment (start 119.38 53.848) (end 122.358002 50.869998) (width 1) (layer B.Cu) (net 9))
 (segment (start 154.94 62.23) (end 154.94 60.96) (width 1) (layer B.Cu) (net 9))
 (segment (start 152.4 64.77) (end 154.94 62.23) (width 1) (layer B.Cu) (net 9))
 (segment (start 154.94 60.96) (end 152.4 60.96) (width 1) (layer B.Cu) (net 9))
 (segment (start 149.86 58.42) (end 149.86 54.61) (width 1) (layer B.Cu) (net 9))
 (segment (start 152.4 60.96) (end 149.86 58.42) (width 1) (layer B.Cu) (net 9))
 (segment (start 160.02 60.96) (end 154.94 60.96) (width 1) (layer B.Cu) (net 9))
 (segment (start 157.48 54.61) (end 161.29 54.61) (width 1) (layer B.Cu) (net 9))
 (segment (start 161.29 60.96) (end 160.02 60.96) (width 1) (layer B.Cu) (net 9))
 (segment (start 162.56 59.69) (end 161.29 60.96) (width 1) (layer B.Cu) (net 9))
 (segment (start 162.56 55.88) (end 162.56 59.69) (width 1) (layer B.Cu) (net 9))
 (segment (start 161.29 54.61) (end 162.56 55.88) (width 1) (layer B.Cu) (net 9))
 (segment (start 153.67 101.6) (end 153.67 100.33) (width 1) (layer B.Cu) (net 16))
 (segment (start 143.57096 97.85096) (end 143.57096 92.71) (width 1) (layer B.Cu) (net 16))
 (segment (start 144.78 99.06) (end 143.57096 97.85096) (width 1) (layer B.Cu) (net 16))
 (segment (start 152.4 99.06) (end 144.78 99.06) (width 1) (layer B.Cu) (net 16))
 (segment (start 153.67 100.33) (end 152.4 99.06) (width 1) (layer B.Cu) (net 16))
 (segment (start 158.75 101.6) (end 158.75 100.33) (width 1) (layer B.Cu) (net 15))
 (segment (start 151.06904 95.18904) (end 151.06904 92.71) (width 1) (layer B.Cu) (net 15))
 (segment (start 152.4 96.52) (end 151.06904 95.18904) (width 1) (layer B.Cu) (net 15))
 (segment (start 154.94 96.52) (end 152.4 96.52) (width 1) (layer B.Cu) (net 15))
 (segment (start 158.75 100.33) (end 154.94 96.52) (width 1) (layer B.Cu) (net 15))
 (segment (start 138.43 101.6) (end 142.24 101.6) (width 1) (layer B.Cu) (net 12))
 (segment (start 116.84 63.5) (end 116.84 58.42) (width 1) (layer B.Cu) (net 11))
 (segment (start 135.89 101.6) (end 135.89 102.87) (width 1) (layer B.Cu) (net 13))
 (segment (start 151.13 102.87) (end 151.13 101.6) (width 1) (layer B.Cu) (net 13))
 (segment (start 149.86 104.14) (end 151.13 102.87) (width 1) (layer B.Cu) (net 13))
 (segment (start 137.16 104.14) (end 149.86 104.14) (width 1) (layer B.Cu) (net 13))
 (segment (start 135.89 102.87) (end 137.16 104.14) (width 1) (layer B.Cu) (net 13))
 (segment (start 127 58.42) (end 127 58.928) (width 1) (layer B.Cu) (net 10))
 (segment (start 127 58.928) (end 129.032 60.96) (width 1) (layer B.Cu) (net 10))
 (segment (start 129.032 60.96) (end 129.96706 60.96) (width 1) (layer B.Cu) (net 10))
 (segment (start 132.08 63.5) (end 132.08 63.07294) (width 1) (layer B.Cu) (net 10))
 (segment (start 132.08 63.07294) (end 129.96706 60.96) (width 1) (layer B.Cu) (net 10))
 (segment (start 127.42706 58.42) (end 127 58.42) (width 1) (layer B.Cu) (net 10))
 (segment (start 144.78 101.6) (end 148.59 101.6) (width 1) (layer B.Cu) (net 14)))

